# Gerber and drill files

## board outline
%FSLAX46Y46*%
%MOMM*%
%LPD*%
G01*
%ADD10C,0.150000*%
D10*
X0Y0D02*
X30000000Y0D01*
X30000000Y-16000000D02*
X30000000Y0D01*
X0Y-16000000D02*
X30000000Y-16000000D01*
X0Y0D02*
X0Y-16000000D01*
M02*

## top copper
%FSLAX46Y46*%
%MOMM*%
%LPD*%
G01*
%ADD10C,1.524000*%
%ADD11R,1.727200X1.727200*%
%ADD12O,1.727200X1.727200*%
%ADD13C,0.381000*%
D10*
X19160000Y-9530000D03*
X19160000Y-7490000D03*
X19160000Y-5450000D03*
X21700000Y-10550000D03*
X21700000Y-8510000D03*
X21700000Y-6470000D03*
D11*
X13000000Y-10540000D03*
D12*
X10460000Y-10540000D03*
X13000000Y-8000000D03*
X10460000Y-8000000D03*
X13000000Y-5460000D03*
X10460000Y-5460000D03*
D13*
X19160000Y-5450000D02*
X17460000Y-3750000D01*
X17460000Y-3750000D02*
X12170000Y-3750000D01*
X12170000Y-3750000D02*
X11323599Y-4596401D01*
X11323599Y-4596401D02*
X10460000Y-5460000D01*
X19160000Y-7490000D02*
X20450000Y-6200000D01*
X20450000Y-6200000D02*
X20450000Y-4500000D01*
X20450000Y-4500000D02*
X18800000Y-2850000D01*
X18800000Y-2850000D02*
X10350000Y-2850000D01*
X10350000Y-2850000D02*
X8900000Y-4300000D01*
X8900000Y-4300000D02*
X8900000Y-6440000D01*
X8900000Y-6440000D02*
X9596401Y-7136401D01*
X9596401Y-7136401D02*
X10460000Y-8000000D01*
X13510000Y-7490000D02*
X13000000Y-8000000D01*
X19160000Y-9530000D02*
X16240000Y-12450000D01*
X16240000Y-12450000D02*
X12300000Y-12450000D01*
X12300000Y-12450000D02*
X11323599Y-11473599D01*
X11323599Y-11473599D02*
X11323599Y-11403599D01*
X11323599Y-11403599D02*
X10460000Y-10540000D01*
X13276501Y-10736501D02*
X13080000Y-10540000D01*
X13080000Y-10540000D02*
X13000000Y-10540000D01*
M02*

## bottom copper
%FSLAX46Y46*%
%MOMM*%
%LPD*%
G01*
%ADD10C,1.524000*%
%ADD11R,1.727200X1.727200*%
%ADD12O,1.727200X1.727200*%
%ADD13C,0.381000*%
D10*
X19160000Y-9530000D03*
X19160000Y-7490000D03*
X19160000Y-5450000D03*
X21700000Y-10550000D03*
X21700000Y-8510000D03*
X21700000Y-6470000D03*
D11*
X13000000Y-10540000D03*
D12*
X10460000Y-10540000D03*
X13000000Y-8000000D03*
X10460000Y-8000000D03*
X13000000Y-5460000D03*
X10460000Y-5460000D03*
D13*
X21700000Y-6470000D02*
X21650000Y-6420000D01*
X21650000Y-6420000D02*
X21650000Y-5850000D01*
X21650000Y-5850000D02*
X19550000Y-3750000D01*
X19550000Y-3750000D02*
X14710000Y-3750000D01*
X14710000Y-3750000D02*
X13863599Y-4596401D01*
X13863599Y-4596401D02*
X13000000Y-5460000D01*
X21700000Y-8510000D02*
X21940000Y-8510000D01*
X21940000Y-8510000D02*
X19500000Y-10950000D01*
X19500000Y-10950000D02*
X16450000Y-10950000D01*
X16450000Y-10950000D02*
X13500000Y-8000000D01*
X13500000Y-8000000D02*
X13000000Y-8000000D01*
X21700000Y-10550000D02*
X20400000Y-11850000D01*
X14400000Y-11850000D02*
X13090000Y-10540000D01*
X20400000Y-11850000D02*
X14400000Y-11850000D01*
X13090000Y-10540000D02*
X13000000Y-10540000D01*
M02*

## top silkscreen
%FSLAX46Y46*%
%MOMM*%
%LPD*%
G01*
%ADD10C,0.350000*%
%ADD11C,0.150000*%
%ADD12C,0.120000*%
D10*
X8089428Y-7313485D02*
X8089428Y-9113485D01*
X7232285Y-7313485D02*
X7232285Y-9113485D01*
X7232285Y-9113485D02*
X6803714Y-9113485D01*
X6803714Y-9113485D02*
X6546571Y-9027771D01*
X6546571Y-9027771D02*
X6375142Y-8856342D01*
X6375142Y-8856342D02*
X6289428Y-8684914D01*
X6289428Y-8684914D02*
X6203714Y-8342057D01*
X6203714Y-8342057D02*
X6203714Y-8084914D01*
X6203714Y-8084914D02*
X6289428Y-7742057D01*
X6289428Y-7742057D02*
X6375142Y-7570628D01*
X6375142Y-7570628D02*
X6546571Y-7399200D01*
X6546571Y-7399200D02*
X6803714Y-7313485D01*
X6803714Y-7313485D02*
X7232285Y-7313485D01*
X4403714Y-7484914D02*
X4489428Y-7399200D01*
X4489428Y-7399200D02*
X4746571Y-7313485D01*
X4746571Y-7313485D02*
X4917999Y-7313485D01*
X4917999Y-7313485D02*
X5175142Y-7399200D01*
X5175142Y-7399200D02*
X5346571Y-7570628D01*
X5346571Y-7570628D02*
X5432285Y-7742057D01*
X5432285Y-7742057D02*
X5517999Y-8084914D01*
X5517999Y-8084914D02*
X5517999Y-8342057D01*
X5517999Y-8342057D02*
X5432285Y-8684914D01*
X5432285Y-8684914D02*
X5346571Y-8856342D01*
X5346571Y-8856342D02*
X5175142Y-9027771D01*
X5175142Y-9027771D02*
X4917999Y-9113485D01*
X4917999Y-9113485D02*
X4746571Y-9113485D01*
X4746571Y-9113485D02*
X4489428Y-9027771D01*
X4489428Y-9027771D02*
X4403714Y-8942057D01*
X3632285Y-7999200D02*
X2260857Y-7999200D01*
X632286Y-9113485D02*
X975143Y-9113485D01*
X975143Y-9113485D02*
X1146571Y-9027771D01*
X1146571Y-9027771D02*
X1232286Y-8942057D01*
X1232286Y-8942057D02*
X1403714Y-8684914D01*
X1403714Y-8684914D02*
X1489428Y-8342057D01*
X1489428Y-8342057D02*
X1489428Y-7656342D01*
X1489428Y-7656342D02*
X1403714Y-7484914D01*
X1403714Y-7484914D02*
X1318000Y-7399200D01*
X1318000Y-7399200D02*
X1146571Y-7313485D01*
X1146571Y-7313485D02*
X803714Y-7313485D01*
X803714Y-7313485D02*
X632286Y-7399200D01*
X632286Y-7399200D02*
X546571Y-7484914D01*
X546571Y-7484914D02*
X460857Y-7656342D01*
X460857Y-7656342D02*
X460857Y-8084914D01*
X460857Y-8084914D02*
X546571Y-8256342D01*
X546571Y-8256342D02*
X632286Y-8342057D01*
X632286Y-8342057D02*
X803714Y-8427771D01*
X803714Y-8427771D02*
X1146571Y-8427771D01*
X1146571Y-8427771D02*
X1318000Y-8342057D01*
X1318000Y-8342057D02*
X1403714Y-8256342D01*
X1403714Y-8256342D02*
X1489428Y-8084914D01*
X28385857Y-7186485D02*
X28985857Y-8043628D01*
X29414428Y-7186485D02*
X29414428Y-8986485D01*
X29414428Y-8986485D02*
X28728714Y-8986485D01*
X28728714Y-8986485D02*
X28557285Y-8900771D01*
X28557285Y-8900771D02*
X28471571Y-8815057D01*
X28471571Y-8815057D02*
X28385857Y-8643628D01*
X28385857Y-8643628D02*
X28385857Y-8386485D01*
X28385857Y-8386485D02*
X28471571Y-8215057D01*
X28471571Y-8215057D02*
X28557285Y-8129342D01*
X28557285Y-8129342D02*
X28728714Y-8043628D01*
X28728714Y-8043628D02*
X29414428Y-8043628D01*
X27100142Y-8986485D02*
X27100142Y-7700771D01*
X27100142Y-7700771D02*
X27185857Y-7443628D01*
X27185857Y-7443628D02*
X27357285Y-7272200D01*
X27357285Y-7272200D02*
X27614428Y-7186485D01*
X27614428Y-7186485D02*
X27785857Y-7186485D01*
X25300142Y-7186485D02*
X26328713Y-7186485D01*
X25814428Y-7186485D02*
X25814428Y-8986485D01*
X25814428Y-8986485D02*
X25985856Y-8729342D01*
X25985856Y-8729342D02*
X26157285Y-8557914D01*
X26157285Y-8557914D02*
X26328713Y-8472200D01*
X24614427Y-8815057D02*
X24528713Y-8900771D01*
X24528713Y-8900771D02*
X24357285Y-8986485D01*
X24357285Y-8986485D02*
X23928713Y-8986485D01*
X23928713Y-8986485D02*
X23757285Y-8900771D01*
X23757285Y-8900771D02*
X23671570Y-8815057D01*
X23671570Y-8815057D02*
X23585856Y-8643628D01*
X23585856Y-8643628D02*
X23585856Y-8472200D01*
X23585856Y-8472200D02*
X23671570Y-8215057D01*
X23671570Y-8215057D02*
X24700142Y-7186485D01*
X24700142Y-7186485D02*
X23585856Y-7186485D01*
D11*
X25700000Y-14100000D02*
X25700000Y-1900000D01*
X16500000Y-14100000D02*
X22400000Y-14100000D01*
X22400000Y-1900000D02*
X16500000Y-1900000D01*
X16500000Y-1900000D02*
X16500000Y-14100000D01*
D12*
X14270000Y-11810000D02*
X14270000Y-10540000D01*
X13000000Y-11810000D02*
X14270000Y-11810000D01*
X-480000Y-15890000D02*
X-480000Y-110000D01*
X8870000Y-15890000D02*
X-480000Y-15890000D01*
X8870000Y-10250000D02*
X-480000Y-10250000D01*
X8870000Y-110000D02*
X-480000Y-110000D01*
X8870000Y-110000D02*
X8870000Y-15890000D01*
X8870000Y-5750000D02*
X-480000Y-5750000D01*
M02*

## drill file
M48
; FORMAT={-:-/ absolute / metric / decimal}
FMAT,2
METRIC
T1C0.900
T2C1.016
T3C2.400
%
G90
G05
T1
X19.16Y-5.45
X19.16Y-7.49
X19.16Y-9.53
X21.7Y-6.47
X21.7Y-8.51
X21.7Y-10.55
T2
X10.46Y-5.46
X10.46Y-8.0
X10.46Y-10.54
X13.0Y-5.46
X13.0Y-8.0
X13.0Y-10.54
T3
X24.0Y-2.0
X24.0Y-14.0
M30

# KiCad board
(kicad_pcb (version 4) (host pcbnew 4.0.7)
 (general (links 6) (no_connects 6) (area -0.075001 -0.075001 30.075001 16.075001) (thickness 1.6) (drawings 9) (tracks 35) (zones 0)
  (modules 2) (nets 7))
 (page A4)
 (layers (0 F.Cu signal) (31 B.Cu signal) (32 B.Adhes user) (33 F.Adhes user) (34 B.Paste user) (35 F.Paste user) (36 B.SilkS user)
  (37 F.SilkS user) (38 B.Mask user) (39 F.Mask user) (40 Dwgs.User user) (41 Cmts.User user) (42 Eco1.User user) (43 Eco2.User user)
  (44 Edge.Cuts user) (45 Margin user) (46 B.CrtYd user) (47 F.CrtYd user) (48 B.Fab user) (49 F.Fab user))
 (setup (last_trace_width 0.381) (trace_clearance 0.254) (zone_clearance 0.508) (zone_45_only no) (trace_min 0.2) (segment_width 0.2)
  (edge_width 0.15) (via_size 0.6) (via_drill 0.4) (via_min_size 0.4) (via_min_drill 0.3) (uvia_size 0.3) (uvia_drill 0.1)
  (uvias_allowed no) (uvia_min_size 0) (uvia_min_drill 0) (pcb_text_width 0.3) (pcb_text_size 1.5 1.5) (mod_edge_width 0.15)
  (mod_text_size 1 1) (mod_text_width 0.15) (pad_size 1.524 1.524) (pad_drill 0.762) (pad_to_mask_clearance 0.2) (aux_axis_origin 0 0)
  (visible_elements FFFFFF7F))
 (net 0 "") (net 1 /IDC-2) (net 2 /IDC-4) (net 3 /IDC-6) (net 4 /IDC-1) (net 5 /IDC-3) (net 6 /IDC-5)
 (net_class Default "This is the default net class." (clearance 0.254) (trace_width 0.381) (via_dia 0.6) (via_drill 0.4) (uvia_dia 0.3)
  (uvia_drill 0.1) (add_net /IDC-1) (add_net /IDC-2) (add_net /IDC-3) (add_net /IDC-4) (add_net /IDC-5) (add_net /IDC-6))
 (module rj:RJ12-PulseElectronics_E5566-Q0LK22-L (layer F.Cu) (at 24 8 90)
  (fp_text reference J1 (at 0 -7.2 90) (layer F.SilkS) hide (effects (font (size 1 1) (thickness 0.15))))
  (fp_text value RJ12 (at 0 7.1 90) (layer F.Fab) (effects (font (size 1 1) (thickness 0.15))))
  (fp_line (start -6.1 1.7) (end 6.1 1.7) (layer F.SilkS) (width 0.15))
  (fp_line (start -6.1 -7.5) (end -6.1 -1.6) (layer F.SilkS) (width 0.15))
  (fp_line (start 6.1 -1.6) (end 6.1 -7.5) (layer F.SilkS) (width 0.15))
  (fp_line (start 6.1 -7.5) (end -6.1 -7.5) (layer F.SilkS) (width 0.15))
  (pad "" np_thru_hole circle (at 6 0 90) (size 2.4 2.4) (drill 2.4) (layers *.Cu *.Mask))
  (pad 5 thru_hole circle (at -1.53 -4.84 90) (size 1.524 1.524) (drill 0.9) (layers *.Cu *.Mask) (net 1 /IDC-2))
  (pad "" np_thru_hole circle (at -6 0 90) (size 2.4 2.4) (drill 2.4) (layers *.Cu *.Mask))
  (pad 3 thru_hole circle (at 0.51 -4.84 90) (size 1.524 1.524) (drill 0.9) (layers *.Cu *.Mask) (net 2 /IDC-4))
  (pad 1 thru_hole circle (at 2.55 -4.84 90) (size 1.524 1.524) (drill 0.9) (layers *.Cu *.Mask) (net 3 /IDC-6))
  (pad 6 thru_hole circle (at -2.55 -2.3 90) (size 1.524 1.524) (drill 0.9) (layers *.Cu *.Mask) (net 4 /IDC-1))
  (pad 4 thru_hole circle (at -0.51 -2.3 90) (size 1.524 1.524) (drill 0.9) (layers *.Cu *.Mask) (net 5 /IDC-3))
  (pad 2 thru_hole circle (at 1.53 -2.3 90) (size 1.524 1.524) (drill 0.9) (layers *.Cu *.Mask) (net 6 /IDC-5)))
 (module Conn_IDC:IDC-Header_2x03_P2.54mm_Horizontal (layer F.Cu) (at 13 10.54 180)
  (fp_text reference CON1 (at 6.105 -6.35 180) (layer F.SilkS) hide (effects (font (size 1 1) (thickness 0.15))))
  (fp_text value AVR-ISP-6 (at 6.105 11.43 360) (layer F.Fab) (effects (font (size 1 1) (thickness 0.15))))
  (fp_line (start -1.27 -1.27) (end -1.27 0) (layer F.SilkS) (width 0.12))
  (fp_line (start 0 -1.27) (end -1.27 -1.27) (layer F.SilkS) (width 0.12))
  (fp_line (start 13.48 -5.35) (end 13.48 10.43) (layer F.SilkS) (width 0.12))
  (fp_line (start 4.13 -5.35) (end 13.48 -5.35) (layer F.SilkS) (width 0.12))
  (fp_line (start 4.13 0.29) (end 13.48 0.29) (layer F.SilkS) (width 0.12))
  (fp_line (start 4.13 10.43) (end 13.48 10.43) (layer F.SilkS) (width 0.12))
  (fp_line (start 4.13 10.43) (end 4.13 -5.35) (layer F.SilkS) (width 0.12))
  (fp_line (start 4.13 4.79) (end 13.48 4.79) (layer F.SilkS) (width 0.12))
  (pad 1 thru_hole rect (at 0 0 180) (size 1.7272 1.7272) (drill 1.016) (layers *.Cu *.Mask) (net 4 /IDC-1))
  (pad 2 thru_hole oval (at 2.54 0 180) (size 1.7272 1.7272) (drill 1.016) (layers *.Cu *.Mask) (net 1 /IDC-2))
  (pad 3 thru_hole oval (at 0 2.54 180) (size 1.7272 1.7272) (drill 1.016) (layers *.Cu *.Mask) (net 5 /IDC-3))
  (pad 4 thru_hole oval (at 2.54 2.54 180) (size 1.7272 1.7272) (drill 1.016) (layers *.Cu *.Mask) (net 2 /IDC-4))
  (pad 5 thru_hole oval (at 0 5.08 180) (size 1.7272 1.7272) (drill 1.016) (layers *.Cu *.Mask) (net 6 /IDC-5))
  (pad 6 thru_hole oval (at 2.54 5.08 180) (size 1.7272 1.7272) (drill 1.016) (layers *.Cu *.Mask) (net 3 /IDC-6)))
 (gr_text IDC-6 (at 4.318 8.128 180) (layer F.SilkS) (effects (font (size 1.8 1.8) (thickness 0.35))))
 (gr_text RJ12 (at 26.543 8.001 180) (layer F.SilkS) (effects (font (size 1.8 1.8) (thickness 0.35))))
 (gr_line (start 0 0) (end 30 0) (layer Edge.Cuts) (width 0.15))
 (gr_line (start 30 16) (end 30 0) (layer Edge.Cuts) (width 0.15))
 (gr_line (start 0 16) (end 30 16) (layer Edge.Cuts) (width 0.15))
 (gr_line (start 0 0) (end 0 16) (layer Edge.Cuts) (width 0.15))
 (segment (start 19.16 5.45) (end 17.46 3.75) (width 0.381) (layer F.Cu) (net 3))
 (segment (start 17.46 3.75) (end 12.17 3.75) (width 0.381) (layer F.Cu) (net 3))
 (segment (start 12.17 3.75) (end 11.323599 4.596401) (width 0.381) (layer F.Cu) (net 3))
 (segment (start 11.323599 4.596401) (end 10.46 5.46) (width 0.381) (layer F.Cu) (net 3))
 (segment (start 21.7 6.47) (end 21.65 6.42) (width 0.381) (layer B.Cu) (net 6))
 (segment (start 21.65 6.42) (end 21.65 5.85) (width 0.381) (layer B.Cu) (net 6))
 (segment (start 21.65 5.85) (end 19.55 3.75) (width 0.381) (layer B.Cu) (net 6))
 (segment (start 19.55 3.75) (end 14.71 3.75) (width 0.381) (layer B.Cu) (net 6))
 (segment (start 14.71 3.75) (end 13.863599 4.596401) (width 0.381) (layer B.Cu) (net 6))
 (segment (start 13.863599 4.596401) (end 13 5.46) (width 0.381) (layer B.Cu) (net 6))
 (segment (start 19.16 7.49) (end 20.45 6.2) (width 0.381) (layer F.Cu) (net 2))
 (segment (start 20.45 6.2) (end 20.45 4.5) (width 0.381) (layer F.Cu) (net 2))
 (segment (start 20.45 4.5) (end 18.8 2.85) (width 0.381) (layer F.Cu) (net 2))
 (segment (start 18.8 2.85) (end 10.35 2.85) (width 0.381) (layer F.Cu) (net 2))
 (segment (start 10.35 2.85) (end 8.9 4.3) (width 0.381) (layer F.Cu) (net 2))
 (segment (start 8.9 4.3) (end 8.9 6.44) (width 0.381) (layer F.Cu) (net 2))
 (segment (start 8.9 6.44) (end 9.596401 7.136401) (width 0.381) (layer F.Cu) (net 2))
 (segment (start 9.596401 7.136401) (end 10.46 8) (width 0.381) (layer F.Cu) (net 2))
 (segment (start 21.7 8.51) (end 21.94 8.51) (width 0.381) (layer B.Cu) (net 5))
 (segment (start 21.94 8.51) (end 19.5 10.95) (width 0.381) (layer B.Cu) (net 5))
 (segment (start 19.5 10.95) (end 16.45 10.95) (width 0.381) (layer B.Cu) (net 5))
 (segment (start 16.45 10.95) (end 13.5 8) (width 0.381) (layer B.Cu) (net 5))
 (segment (start 13.5 8) (end 13 8) (width 0.381) (layer B.Cu) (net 5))
 (segment (start 13.51 7.49) (end 13 8) (width 0.381) (layer F.Cu) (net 5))
 (segment (start 19.16 9.53) (end 16.24 12.45) (width 0.381) (layer F.Cu) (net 1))
 (segment (start 16.24 12.45) (end 12.3 12.45) (width 0.381) (layer F.Cu) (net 1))
 (segment (start 12.3 12.45) (end 11.323599 11.473599) (width 0.381) (layer F.Cu) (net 1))
 (segment (start 11.323599 11.473599) (end 11.323599 11.403599) (width 0.381) (layer F.Cu) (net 1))
 (segment (start 11.323599 11.403599) (end 10.46 10.54) (width 0.381) (layer F.Cu) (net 1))
 (segment (start 21.7 10.55) (end 20.4 11.85) (width 0.381) (layer B.Cu) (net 4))
 (segment (start 14.4 11.85) (end 13.09 10.54) (width 0.381) (layer B.Cu) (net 4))
 (segment (start 20.4 11.85) (end 14.4 11.85) (width 0.381) (layer B.Cu) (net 4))
 (segment (start 13.09 10.54) (end 13 10.54) (width 0.381) (layer B.Cu) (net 4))
 (segment (start 13.276501 10.736501) (end 13.08 10.54) (width 0.381) (layer F.Cu) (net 4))
 (segment (start 13.08 10.54) (end 13 10.54) (width 0.381) (layer F.Cu) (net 4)))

